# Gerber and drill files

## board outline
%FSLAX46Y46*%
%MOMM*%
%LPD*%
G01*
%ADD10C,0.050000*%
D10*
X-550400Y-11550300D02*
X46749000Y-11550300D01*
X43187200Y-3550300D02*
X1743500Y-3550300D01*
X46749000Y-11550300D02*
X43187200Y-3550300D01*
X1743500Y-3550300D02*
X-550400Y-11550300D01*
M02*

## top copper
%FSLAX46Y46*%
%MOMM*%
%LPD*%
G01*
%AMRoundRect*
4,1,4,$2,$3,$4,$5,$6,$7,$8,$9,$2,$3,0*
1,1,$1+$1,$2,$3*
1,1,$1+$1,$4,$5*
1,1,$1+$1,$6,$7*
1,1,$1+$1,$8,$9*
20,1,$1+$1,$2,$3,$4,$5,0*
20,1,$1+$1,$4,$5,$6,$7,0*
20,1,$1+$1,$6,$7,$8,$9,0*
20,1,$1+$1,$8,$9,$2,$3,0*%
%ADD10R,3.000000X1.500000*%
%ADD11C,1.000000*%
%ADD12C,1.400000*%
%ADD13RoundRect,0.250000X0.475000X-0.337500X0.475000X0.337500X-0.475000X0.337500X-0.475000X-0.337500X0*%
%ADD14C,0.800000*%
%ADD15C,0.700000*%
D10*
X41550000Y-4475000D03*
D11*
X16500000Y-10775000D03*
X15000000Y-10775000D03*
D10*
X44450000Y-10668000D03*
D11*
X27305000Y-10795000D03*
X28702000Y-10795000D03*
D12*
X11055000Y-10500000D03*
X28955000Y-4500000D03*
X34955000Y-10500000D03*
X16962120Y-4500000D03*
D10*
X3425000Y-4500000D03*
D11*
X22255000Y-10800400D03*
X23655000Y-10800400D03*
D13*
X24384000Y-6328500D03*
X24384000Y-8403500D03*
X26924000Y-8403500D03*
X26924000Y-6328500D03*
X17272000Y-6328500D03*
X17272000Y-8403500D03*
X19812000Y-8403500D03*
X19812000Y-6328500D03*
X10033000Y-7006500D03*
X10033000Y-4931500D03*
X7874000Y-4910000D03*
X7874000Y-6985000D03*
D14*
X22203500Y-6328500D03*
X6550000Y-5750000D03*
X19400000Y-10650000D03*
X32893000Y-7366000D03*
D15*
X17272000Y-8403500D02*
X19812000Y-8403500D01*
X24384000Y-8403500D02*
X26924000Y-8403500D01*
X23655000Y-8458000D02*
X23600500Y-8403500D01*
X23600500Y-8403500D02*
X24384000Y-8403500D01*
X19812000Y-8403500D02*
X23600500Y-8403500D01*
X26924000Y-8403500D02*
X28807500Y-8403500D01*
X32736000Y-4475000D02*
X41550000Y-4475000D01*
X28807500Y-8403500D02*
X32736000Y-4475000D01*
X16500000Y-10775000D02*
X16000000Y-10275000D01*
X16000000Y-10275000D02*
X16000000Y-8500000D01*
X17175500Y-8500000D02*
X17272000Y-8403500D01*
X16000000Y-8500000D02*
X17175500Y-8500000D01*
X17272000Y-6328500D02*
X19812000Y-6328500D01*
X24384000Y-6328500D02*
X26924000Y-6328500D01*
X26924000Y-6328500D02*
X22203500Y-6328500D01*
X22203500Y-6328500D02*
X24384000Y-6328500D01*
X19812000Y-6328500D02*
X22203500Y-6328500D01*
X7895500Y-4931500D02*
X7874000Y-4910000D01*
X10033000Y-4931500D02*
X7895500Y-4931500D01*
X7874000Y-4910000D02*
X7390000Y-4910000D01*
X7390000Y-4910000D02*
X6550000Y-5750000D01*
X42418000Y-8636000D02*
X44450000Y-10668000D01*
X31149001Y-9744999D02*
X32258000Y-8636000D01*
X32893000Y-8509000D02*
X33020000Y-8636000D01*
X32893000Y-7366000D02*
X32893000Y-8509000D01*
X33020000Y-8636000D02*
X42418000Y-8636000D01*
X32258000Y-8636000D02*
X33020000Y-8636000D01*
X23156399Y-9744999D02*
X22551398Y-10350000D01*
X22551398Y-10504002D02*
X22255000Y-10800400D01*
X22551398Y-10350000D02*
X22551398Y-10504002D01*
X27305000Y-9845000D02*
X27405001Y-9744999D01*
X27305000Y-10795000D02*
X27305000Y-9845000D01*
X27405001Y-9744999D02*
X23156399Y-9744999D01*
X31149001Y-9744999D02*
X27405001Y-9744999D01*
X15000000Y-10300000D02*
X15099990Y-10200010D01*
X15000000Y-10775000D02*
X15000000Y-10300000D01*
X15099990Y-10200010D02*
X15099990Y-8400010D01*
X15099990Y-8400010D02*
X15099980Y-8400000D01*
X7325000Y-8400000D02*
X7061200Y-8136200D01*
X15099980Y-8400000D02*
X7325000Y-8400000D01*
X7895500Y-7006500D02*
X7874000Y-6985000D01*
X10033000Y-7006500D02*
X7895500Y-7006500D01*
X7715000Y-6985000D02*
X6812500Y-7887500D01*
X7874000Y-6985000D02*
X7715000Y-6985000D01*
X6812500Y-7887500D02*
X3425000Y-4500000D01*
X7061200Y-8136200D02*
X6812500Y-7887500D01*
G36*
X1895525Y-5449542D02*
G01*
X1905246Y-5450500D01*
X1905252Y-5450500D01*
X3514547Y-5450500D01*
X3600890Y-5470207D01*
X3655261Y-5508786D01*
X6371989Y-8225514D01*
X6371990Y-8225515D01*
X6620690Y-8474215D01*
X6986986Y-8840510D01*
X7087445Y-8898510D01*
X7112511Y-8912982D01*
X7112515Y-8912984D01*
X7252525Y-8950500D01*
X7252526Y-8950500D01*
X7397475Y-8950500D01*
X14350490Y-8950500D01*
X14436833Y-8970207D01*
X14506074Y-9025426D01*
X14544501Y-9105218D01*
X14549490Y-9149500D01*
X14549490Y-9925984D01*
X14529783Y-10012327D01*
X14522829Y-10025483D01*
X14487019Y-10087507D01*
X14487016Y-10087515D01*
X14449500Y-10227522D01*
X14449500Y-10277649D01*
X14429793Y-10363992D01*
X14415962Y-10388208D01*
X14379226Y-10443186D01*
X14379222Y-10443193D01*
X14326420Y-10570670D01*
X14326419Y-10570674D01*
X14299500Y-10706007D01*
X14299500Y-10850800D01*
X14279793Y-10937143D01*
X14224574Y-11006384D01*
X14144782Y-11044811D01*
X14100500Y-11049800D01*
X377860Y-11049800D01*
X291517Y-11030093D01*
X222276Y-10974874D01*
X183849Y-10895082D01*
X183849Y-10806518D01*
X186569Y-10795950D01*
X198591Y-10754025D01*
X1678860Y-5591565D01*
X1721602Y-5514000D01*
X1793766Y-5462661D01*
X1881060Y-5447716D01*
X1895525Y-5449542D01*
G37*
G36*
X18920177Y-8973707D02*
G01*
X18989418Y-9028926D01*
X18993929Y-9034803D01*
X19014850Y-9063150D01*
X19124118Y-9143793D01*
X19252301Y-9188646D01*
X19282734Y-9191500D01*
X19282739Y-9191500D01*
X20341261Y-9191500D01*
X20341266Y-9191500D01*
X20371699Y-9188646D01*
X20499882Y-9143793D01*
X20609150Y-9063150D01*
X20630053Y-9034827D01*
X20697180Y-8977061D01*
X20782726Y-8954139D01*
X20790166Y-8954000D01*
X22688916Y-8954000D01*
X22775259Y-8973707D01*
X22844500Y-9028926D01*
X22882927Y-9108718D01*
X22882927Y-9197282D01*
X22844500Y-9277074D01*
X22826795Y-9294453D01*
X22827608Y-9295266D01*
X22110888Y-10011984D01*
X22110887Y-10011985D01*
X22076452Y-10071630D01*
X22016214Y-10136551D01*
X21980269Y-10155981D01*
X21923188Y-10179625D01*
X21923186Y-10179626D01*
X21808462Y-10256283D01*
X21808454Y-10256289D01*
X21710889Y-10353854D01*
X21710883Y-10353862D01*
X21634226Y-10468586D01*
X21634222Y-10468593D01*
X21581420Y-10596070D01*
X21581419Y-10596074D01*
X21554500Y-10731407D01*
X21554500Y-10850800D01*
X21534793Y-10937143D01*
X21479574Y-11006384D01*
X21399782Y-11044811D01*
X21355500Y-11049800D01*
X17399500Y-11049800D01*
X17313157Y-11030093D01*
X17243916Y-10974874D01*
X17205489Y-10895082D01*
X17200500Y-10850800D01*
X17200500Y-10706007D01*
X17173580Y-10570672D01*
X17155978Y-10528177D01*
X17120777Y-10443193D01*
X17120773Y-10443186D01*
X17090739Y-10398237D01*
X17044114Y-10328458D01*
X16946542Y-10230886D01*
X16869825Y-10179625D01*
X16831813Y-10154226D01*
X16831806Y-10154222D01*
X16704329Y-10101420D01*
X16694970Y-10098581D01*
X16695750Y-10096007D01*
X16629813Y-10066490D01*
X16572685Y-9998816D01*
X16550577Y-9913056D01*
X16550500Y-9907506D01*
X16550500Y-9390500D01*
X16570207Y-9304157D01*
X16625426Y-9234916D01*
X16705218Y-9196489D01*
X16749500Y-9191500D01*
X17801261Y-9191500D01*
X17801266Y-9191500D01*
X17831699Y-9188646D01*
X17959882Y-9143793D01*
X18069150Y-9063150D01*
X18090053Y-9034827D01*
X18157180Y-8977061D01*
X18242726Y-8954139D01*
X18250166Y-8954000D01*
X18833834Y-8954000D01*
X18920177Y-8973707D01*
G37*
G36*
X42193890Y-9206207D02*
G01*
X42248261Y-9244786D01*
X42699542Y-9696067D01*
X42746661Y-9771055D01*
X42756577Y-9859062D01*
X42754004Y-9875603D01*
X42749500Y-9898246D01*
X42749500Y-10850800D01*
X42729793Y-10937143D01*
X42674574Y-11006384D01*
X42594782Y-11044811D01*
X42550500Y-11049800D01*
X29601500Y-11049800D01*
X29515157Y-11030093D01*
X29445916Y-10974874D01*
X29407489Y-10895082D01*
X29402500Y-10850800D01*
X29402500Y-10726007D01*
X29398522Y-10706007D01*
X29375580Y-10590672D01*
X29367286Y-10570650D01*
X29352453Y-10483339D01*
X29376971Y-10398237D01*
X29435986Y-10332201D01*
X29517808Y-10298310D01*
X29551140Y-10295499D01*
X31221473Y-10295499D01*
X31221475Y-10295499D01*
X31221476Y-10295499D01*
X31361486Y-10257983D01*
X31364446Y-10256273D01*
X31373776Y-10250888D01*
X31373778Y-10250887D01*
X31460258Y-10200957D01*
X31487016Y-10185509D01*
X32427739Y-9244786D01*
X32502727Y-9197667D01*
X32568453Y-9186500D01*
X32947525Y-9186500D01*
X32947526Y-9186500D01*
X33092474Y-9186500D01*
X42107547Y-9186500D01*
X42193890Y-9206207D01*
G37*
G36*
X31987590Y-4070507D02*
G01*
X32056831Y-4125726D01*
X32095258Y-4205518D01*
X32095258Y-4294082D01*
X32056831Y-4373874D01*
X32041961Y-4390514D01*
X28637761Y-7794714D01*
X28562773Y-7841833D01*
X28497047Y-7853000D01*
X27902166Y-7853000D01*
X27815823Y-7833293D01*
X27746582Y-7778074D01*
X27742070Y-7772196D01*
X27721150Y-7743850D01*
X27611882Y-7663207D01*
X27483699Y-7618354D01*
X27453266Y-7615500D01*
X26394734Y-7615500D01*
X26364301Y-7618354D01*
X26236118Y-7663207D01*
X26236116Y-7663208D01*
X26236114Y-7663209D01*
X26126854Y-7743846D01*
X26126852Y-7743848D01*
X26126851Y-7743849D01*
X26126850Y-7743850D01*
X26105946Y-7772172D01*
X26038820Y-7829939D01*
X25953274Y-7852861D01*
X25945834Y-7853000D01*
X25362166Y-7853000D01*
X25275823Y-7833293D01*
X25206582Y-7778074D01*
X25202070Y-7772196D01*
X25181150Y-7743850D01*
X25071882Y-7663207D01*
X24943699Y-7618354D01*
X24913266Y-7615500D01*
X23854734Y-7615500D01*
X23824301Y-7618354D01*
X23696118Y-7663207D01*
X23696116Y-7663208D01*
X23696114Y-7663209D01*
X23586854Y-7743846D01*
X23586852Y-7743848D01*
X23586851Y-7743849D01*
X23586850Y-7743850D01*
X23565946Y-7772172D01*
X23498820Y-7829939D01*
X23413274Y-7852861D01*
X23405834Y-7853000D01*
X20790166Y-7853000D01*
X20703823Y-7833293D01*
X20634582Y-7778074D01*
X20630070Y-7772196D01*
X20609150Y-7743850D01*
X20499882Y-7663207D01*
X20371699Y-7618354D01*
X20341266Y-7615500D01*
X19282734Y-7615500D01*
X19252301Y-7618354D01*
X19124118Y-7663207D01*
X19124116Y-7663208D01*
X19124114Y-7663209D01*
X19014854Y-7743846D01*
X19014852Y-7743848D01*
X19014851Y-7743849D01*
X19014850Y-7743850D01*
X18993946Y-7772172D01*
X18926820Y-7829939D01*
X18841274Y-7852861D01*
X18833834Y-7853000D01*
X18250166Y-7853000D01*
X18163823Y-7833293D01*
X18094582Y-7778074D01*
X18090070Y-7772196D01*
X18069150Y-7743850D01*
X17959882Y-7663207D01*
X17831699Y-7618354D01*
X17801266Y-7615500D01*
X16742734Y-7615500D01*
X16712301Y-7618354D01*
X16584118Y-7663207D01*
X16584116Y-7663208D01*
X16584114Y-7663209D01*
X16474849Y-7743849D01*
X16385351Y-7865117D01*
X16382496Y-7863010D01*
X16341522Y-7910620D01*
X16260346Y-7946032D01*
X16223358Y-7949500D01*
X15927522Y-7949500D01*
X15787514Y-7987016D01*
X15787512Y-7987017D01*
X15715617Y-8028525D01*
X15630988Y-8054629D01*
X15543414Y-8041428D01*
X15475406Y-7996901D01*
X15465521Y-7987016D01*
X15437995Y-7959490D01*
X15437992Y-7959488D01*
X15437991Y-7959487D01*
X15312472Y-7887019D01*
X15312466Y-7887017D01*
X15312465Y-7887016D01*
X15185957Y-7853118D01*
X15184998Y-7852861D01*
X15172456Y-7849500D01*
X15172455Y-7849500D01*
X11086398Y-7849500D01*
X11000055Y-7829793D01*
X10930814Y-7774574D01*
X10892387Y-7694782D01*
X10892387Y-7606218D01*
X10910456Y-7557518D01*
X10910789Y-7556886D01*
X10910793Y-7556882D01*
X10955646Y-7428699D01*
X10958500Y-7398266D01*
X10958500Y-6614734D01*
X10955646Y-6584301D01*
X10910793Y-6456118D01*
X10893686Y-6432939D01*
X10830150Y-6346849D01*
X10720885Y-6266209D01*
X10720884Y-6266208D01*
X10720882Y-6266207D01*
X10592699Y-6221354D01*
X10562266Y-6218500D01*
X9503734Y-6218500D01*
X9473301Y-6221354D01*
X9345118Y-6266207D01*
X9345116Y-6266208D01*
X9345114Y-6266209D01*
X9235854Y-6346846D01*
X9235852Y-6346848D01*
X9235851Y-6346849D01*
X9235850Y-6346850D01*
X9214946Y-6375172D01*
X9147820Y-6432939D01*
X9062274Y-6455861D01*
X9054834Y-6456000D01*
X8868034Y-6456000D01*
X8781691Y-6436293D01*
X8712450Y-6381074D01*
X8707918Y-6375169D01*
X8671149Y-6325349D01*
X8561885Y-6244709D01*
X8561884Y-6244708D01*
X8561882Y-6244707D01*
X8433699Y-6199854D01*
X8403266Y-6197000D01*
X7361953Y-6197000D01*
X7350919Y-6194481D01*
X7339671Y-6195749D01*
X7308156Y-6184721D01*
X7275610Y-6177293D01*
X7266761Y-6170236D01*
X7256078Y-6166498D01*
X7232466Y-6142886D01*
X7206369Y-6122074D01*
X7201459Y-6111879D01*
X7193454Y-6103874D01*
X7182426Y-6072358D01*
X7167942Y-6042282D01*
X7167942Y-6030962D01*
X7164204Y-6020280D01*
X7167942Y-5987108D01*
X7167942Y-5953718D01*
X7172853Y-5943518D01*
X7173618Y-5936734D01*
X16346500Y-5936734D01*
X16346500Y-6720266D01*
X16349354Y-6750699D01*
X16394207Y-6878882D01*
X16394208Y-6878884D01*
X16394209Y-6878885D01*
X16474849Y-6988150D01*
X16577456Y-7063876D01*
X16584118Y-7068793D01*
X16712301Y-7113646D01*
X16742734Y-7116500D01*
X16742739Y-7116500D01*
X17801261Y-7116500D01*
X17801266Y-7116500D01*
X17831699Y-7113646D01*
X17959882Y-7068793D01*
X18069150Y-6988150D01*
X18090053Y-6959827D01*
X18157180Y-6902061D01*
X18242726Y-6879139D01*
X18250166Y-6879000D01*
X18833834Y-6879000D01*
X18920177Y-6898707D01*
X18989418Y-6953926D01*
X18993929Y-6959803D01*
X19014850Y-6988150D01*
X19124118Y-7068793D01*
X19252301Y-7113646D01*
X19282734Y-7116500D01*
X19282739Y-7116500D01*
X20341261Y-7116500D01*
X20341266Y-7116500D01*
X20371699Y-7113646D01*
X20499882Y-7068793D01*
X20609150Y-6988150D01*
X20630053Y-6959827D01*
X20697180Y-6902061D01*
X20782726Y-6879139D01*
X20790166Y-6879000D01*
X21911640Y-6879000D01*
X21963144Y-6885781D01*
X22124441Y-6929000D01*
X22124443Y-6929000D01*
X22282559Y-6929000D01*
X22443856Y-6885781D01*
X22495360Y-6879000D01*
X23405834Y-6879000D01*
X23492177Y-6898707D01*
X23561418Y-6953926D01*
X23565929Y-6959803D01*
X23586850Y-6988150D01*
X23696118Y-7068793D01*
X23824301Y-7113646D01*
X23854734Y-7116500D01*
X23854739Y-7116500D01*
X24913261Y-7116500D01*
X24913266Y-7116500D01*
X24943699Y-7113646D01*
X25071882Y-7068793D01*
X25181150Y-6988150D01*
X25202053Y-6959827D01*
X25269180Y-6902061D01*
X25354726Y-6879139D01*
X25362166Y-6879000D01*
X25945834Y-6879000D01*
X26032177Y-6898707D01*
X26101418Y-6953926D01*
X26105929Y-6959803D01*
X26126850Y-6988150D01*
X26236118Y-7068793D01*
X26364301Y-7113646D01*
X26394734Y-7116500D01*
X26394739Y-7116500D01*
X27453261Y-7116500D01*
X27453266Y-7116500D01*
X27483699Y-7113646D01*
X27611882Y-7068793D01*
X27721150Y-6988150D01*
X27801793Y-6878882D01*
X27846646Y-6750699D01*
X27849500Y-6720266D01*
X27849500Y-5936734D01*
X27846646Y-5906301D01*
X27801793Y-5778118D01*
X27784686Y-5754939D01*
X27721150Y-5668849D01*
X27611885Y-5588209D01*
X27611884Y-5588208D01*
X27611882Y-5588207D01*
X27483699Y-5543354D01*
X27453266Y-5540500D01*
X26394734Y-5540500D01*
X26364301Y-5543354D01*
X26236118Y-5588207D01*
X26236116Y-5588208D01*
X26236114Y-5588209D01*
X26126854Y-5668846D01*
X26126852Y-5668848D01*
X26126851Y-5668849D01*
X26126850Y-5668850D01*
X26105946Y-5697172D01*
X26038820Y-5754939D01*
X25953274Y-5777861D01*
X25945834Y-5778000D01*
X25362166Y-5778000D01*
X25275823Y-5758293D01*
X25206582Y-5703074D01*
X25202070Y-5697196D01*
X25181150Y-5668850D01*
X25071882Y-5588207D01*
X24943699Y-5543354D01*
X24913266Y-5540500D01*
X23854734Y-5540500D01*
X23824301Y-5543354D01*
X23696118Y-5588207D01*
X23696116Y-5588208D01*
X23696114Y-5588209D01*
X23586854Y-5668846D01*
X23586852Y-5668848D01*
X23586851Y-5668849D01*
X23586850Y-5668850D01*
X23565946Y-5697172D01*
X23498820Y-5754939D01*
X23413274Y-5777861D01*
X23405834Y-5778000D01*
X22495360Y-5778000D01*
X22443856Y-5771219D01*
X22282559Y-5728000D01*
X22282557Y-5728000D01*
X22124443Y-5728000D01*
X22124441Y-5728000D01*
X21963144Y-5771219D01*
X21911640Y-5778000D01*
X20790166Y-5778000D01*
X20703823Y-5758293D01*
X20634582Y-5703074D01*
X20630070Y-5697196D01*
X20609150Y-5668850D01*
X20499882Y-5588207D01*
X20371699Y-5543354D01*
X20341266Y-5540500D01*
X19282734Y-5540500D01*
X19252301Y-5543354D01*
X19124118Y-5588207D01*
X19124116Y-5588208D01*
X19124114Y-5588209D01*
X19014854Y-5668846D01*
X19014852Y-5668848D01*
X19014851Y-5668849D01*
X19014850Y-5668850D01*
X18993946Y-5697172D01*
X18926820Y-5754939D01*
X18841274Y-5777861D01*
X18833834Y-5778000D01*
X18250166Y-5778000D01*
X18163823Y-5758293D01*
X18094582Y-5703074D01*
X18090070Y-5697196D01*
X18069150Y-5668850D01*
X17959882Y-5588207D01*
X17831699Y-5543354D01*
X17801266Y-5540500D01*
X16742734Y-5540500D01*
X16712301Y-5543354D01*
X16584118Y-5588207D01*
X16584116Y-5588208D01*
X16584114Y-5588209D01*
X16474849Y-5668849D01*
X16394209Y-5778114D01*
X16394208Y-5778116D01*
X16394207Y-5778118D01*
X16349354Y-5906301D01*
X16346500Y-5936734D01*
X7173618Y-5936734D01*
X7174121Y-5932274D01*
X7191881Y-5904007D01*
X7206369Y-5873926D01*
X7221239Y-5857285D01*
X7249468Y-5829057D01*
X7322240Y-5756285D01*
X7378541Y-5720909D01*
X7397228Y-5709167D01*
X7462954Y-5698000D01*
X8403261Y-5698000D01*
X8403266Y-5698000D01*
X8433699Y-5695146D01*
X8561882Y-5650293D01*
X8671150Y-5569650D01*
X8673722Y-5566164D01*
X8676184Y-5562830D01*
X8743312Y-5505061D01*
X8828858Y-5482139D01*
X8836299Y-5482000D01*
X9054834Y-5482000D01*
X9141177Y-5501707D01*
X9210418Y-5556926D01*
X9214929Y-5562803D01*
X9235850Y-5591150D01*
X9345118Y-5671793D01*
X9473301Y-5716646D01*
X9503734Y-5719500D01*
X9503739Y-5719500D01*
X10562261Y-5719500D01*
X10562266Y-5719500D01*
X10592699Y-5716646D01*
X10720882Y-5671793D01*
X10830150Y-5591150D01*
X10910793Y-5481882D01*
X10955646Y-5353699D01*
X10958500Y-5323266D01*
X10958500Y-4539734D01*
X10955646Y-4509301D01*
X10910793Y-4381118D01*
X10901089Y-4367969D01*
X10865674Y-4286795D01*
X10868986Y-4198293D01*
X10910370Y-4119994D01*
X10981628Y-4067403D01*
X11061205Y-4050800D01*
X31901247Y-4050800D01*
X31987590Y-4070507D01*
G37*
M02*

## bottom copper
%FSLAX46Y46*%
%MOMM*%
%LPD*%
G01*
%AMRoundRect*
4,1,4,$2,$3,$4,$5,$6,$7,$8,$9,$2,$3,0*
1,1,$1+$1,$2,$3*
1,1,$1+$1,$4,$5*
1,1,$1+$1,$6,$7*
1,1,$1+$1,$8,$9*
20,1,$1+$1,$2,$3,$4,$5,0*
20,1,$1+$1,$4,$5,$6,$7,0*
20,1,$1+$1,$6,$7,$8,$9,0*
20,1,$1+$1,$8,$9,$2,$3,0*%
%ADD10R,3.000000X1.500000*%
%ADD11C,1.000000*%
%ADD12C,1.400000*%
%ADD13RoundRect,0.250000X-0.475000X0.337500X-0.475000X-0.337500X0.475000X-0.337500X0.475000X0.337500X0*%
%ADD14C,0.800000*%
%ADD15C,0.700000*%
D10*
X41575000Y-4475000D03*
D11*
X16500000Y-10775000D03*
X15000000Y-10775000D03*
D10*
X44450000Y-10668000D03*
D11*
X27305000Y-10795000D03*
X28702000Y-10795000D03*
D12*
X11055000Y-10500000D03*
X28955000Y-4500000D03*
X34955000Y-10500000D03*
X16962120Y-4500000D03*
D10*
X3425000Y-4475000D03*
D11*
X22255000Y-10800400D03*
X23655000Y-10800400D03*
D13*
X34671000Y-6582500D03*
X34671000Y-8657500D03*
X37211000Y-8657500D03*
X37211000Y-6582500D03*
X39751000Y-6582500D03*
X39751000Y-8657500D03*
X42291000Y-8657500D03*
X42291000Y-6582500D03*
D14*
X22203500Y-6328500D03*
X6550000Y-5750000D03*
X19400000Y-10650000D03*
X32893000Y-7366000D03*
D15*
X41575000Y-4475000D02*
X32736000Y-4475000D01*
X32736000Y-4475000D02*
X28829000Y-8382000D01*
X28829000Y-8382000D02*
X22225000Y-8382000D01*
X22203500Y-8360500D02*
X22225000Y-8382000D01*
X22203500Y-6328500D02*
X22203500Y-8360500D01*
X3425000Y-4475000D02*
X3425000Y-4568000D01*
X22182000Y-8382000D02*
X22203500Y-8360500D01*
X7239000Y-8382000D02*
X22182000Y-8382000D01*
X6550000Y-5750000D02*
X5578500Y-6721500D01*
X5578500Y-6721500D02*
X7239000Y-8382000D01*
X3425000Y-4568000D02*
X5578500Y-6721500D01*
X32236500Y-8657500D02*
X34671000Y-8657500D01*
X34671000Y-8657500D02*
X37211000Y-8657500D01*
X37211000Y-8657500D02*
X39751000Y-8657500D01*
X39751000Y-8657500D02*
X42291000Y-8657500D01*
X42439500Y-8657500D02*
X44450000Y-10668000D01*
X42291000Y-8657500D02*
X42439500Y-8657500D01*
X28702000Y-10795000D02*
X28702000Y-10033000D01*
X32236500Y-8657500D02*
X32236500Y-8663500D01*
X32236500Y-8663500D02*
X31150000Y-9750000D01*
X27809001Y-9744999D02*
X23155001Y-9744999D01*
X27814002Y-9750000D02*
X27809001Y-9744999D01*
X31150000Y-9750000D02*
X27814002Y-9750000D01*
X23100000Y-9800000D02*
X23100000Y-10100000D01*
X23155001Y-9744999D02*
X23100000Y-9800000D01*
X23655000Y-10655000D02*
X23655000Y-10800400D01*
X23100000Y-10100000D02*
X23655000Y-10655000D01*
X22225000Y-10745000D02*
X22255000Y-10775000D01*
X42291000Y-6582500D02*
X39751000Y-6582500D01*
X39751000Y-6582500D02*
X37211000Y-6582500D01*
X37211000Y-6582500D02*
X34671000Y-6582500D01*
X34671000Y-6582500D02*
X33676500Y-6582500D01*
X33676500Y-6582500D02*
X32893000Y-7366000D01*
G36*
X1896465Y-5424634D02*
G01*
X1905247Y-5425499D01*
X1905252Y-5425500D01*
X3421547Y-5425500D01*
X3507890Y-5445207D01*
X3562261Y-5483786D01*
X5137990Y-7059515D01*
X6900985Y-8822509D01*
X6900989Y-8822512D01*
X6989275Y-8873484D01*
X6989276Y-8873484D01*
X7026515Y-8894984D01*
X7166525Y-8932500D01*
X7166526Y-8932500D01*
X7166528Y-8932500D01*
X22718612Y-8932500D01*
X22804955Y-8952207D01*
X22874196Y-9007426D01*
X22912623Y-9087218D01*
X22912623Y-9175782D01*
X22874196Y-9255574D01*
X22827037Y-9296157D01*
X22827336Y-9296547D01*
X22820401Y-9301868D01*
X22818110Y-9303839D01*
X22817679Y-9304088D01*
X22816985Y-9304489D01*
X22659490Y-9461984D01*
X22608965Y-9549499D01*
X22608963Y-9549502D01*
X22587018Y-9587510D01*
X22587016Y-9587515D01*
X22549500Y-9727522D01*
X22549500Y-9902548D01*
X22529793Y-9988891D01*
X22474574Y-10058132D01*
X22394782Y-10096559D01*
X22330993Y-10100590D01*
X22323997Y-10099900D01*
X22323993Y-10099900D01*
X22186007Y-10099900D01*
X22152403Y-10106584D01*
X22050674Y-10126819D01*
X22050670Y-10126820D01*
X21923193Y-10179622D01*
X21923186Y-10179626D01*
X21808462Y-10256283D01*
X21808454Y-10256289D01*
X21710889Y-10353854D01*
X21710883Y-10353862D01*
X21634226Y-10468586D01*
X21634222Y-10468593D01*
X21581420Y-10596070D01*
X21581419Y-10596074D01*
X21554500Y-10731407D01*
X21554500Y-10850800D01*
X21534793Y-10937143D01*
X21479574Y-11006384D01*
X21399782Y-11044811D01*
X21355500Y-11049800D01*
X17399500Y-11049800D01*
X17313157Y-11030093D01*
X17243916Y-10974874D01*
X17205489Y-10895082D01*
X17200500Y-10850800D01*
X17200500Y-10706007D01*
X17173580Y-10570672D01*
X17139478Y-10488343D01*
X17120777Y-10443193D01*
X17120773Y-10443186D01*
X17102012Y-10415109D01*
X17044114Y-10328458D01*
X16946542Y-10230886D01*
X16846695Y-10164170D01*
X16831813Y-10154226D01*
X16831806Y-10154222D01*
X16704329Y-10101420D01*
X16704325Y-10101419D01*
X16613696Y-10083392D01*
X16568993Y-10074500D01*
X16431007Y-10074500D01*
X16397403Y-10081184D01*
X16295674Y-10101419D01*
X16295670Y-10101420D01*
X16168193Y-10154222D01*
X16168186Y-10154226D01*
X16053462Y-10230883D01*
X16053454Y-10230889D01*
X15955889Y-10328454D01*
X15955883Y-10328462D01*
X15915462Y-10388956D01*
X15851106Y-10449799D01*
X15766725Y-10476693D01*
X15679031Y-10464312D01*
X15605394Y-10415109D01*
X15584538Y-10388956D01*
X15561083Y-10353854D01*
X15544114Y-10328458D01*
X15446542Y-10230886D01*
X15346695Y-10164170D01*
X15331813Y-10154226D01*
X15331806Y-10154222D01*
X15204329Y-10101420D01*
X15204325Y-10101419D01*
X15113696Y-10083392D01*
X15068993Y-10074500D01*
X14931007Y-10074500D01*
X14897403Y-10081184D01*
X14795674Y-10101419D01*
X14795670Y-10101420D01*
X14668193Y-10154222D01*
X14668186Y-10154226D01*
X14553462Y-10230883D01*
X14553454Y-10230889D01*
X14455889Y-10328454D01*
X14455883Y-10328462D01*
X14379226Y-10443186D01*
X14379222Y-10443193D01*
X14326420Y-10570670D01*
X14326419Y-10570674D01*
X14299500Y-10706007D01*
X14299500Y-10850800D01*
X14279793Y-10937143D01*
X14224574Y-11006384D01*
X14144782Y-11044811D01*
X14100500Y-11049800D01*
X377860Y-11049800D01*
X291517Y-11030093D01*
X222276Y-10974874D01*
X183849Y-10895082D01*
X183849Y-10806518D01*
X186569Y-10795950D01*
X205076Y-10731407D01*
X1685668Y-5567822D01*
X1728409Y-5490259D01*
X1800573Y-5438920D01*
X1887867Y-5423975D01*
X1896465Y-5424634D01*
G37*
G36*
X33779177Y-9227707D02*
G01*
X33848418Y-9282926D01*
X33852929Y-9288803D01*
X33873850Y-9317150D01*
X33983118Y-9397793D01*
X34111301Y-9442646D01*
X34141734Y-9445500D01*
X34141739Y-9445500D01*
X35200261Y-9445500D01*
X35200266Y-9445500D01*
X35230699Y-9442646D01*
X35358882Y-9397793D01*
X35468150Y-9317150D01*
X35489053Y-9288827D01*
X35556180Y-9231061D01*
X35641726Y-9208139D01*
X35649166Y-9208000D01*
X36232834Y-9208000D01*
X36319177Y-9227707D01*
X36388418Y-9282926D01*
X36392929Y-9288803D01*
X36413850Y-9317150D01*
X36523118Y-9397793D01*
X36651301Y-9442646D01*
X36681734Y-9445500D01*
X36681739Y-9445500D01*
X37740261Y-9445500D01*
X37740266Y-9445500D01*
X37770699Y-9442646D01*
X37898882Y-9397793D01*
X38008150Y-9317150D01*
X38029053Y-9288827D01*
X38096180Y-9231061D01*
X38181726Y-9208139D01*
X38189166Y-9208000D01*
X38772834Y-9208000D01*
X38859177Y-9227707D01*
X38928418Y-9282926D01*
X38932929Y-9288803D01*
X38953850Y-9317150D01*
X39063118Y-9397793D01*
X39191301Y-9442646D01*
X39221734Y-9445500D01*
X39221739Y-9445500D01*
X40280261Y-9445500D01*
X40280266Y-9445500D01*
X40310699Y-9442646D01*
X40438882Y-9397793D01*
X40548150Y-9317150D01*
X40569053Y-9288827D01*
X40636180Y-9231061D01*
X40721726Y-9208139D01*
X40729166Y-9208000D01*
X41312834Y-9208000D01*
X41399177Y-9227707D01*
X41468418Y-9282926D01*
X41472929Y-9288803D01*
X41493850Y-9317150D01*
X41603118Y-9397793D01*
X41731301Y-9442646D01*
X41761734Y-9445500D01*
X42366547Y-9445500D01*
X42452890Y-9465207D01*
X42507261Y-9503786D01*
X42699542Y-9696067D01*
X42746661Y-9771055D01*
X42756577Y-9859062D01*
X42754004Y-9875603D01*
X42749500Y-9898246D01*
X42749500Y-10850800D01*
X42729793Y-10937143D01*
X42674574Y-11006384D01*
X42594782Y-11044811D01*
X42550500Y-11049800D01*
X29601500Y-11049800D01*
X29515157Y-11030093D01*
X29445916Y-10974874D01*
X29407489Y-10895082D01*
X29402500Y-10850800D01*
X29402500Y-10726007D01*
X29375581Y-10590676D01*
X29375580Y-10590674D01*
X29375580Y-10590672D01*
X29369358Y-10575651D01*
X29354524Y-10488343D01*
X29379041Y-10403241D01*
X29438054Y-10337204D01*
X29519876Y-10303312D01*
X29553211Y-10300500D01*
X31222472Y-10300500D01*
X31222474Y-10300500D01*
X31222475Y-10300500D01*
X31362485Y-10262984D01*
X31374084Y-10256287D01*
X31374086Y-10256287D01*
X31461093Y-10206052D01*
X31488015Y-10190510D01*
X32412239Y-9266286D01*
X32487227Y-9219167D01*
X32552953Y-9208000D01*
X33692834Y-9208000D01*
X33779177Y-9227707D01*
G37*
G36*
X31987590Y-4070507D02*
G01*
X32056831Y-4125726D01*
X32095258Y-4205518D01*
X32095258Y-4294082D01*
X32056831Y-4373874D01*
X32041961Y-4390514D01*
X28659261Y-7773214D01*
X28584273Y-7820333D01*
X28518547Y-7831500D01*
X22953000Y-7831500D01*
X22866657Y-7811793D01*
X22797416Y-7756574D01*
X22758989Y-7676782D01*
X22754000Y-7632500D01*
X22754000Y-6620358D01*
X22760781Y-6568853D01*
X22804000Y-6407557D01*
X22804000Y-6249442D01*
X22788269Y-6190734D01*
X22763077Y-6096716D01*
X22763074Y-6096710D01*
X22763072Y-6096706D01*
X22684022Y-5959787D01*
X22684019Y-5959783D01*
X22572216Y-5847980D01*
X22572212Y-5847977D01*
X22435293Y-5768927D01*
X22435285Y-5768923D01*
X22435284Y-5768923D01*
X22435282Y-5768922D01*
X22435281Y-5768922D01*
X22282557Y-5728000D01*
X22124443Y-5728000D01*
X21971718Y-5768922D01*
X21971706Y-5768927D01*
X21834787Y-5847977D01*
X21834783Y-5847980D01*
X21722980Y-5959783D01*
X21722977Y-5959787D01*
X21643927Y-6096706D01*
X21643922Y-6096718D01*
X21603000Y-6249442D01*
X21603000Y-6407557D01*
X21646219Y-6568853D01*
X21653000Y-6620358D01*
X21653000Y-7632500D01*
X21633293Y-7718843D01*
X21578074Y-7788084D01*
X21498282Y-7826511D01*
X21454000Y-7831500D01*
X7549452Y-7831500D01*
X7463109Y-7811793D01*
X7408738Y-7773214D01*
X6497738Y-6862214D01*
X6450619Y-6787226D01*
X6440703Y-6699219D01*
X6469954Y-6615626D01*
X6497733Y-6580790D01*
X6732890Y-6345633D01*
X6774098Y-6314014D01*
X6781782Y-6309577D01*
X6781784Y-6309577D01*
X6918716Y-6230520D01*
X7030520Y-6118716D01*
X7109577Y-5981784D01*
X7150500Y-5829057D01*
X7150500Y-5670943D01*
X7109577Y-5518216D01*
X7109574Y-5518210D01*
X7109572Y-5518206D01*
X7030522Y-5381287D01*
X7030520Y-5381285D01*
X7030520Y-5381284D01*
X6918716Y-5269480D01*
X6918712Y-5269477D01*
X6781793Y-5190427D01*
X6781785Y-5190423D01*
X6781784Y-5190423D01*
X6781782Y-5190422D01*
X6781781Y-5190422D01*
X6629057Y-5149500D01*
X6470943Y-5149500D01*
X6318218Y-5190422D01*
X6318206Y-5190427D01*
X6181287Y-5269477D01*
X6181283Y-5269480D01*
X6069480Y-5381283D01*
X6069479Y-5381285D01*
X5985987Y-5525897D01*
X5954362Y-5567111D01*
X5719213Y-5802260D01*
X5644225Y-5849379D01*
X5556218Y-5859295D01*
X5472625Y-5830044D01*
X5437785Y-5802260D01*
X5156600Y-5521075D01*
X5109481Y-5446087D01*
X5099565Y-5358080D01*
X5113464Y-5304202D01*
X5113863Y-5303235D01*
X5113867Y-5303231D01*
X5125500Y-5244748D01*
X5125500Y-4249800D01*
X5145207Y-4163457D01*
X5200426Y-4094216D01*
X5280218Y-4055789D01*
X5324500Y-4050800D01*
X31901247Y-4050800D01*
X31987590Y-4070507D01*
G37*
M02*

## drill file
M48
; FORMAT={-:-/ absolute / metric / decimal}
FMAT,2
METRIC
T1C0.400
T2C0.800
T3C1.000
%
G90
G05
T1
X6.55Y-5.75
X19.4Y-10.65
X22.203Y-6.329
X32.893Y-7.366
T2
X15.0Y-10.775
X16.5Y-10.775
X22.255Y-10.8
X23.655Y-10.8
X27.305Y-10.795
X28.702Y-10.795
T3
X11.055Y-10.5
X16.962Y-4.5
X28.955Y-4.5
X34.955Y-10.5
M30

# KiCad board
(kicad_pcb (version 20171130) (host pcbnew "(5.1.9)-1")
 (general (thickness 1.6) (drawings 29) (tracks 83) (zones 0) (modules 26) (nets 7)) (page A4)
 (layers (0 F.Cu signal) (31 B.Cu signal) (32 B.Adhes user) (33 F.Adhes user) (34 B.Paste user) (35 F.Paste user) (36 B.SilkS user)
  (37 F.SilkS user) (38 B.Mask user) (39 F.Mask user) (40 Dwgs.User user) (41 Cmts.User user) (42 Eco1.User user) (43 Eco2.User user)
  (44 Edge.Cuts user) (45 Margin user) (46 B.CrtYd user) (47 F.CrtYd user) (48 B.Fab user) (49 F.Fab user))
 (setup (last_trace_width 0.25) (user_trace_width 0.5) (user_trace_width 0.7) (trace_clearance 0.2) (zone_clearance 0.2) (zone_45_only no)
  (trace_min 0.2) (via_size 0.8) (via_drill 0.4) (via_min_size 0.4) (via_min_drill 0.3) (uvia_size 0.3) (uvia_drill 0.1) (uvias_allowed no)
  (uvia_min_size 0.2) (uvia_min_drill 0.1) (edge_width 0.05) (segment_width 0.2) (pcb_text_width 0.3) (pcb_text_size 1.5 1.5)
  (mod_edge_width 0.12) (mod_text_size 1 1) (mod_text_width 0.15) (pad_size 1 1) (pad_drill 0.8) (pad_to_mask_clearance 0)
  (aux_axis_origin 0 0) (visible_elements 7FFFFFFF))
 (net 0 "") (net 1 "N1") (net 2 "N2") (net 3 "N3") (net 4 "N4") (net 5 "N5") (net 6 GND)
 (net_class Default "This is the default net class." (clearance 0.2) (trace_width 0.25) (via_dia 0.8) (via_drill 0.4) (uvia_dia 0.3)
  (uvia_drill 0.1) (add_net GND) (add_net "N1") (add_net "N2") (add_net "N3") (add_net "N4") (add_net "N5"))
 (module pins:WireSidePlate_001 (layer F.Cu) (at 41.55 2.275)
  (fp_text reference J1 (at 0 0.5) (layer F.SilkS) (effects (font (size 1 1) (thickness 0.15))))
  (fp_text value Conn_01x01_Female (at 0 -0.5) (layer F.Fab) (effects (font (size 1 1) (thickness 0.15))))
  (pad 1 smd rect (at 0 2.2) (size 3 1.5) (layers F.Cu F.Paste F.Mask) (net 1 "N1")))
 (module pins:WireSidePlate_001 (layer B.Cu) (at 41.575 6.675)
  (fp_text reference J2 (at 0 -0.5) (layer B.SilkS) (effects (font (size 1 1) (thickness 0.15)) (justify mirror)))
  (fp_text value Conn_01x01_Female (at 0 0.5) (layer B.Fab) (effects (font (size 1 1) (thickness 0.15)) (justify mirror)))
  (pad 1 smd rect (at 0 -2.2) (size 3 1.5) (layers B.Cu B.Paste B.Mask) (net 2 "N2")))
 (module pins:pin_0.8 (layer F.Cu) (at 23.655 10.775 270)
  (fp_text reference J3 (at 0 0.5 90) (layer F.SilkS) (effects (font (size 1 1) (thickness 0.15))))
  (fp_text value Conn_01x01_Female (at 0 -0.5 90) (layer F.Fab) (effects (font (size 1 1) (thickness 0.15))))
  (pad 1 thru_hole circle (at 0 7.155 270) (size 1 1) (drill 0.8) (layers *.Cu *.Mask) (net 1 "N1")))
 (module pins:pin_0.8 (layer F.Cu) (at 21.65 10.775 270)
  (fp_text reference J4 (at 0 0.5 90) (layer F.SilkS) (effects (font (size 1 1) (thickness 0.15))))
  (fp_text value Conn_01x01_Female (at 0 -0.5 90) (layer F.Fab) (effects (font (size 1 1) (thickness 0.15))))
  (pad 1 thru_hole circle (at 0 6.65 270) (size 1 1) (drill 0.8) (layers *.Cu *.Mask) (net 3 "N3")))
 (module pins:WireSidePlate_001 (layer F.Cu) (at 44.45 8.468)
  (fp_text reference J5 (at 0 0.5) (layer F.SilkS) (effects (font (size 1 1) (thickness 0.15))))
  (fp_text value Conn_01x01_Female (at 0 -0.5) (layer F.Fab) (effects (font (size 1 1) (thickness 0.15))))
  (pad 1 smd rect (at 0 2.2) (size 3 1.5) (layers F.Cu F.Paste F.Mask) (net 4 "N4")))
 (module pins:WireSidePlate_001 (layer B.Cu) (at 44.45 12.868)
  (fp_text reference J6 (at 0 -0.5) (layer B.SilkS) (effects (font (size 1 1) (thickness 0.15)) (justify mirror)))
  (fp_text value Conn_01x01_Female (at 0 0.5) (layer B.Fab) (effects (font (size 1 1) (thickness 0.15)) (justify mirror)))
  (pad 1 smd rect (at 0 -2.2) (size 3 1.5) (layers B.Cu B.Paste B.Mask) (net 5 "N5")))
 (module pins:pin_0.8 (layer F.Cu) (at 27.305 9.195)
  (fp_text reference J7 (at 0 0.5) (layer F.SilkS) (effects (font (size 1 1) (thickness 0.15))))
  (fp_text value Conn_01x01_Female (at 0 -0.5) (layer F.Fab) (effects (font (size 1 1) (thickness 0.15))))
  (pad 1 thru_hole circle (at 0 1.6) (size 1 1) (drill 0.8) (layers *.Cu *.Mask) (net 4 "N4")))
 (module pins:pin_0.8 (layer F.Cu) (at 28.702 9.195)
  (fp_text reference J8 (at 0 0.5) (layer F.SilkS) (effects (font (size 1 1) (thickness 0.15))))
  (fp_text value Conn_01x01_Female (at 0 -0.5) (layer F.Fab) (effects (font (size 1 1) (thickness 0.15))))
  (pad 1 thru_hole circle (at 0 1.6) (size 1 1) (drill 0.8) (layers *.Cu *.Mask) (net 5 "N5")))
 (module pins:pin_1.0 (layer F.Cu) (at 31.195 22.195)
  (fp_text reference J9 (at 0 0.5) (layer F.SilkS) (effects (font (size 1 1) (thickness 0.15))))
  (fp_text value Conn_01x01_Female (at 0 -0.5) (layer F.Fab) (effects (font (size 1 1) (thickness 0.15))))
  (pad 1 thru_hole circle (at -20.14 -11.695) (size 1.4 1.4) (drill 1) (layers *.Cu *.Mask) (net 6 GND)))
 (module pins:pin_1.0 (layer F.Cu) (at 28.855 2.5)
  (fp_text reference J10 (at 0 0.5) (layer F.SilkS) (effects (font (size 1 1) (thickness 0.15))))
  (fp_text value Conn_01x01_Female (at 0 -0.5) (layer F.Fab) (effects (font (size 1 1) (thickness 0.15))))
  (pad 1 thru_hole circle (at 0.1 2) (size 1.4 1.4) (drill 1) (layers *.Cu *.Mask) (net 6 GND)))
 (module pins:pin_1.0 (layer F.Cu) (at 30.385 26.395)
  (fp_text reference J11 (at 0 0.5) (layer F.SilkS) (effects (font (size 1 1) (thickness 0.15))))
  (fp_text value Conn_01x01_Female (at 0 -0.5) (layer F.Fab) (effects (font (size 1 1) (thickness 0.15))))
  (pad 1 thru_hole circle (at 4.57 -15.895) (size 1.4 1.4) (drill 1) (layers *.Cu *.Mask) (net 6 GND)))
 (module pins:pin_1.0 (layer F.Cu) (at 16.86212 2.5)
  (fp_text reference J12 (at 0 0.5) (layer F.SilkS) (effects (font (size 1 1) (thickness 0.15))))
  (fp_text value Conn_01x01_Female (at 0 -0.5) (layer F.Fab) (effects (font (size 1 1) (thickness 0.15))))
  (pad 1 thru_hole circle (at 0.1 2) (size 1.4 1.4) (drill 1) (layers *.Cu *.Mask) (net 6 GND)))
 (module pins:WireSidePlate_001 (layer F.Cu) (at 3.425 2.3)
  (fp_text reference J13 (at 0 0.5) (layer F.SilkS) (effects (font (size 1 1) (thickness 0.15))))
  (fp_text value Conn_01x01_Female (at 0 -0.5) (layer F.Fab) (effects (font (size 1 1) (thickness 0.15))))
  (pad 1 smd rect (at 0 2.2) (size 3 1.5) (layers F.Cu F.Paste F.Mask) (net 3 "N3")))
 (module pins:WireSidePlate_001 (layer B.Cu) (at 3.425 6.675)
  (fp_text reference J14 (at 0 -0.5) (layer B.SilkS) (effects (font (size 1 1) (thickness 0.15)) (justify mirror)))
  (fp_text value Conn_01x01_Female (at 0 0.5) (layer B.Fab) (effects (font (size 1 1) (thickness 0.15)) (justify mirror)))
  (pad 1 smd rect (at 0 -2.2) (size 3 1.5) (layers B.Cu B.Paste B.Mask) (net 2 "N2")))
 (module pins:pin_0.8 (layer F.Cu) (at 8.45764 9.20068)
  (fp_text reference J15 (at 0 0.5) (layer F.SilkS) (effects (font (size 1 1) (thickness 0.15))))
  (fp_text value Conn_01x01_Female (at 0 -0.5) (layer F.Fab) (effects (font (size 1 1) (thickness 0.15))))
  (pad 1 thru_hole circle (at 13.79736 1.59972) (size 1 1) (drill 0.8) (layers *.Cu *.Mask) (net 4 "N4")))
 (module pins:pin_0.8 (layer F.Cu) (at 7.0612 9.20008)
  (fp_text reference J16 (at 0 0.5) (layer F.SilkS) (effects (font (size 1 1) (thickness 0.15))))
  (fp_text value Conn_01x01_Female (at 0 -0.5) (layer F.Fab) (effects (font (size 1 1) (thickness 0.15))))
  (pad 1 thru_hole circle (at 16.5938 1.60032) (size 1 1) (drill 0.8) (layers *.Cu *.Mask) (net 5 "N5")))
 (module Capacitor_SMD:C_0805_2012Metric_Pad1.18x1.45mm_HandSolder (layer B.Cu) (at 34.671 7.62 270)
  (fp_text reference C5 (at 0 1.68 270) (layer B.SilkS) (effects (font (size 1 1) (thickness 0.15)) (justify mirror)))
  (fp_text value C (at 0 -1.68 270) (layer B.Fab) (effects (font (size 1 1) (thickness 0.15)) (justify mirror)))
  (pad 1 smd roundrect (at -1.0375 0 270) (size 1.175 1.45) (layers B.Cu B.Paste B.Mask) (roundrect_rratio 0.2127659574468085) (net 4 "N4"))
  (pad 2 smd roundrect (at 1.0375 0 270) (size 1.175 1.45) (layers B.Cu B.Paste B.Mask) (roundrect_rratio 0.2127659574468085) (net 5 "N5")))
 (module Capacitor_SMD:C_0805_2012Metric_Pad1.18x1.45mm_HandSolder (layer B.Cu) (at 37.211 7.62 270)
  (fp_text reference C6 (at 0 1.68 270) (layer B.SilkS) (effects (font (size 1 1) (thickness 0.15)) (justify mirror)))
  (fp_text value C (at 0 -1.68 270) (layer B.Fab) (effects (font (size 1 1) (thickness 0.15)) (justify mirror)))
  (pad 2 smd roundrect (at 1.0375 0 270) (size 1.175 1.45) (layers B.Cu B.Paste B.Mask) (roundrect_rratio 0.2127659574468085) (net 5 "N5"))
  (pad 1 smd roundrect (at -1.0375 0 270) (size 1.175 1.45) (layers B.Cu B.Paste B.Mask) (roundrect_rratio 0.2127659574468085) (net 4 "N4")))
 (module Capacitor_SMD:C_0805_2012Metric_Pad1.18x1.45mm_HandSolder (layer B.Cu) (at 39.751 7.62 270)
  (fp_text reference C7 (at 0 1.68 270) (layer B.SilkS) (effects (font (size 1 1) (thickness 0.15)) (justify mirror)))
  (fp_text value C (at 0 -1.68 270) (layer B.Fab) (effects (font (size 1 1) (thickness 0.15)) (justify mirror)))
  (pad 1 smd roundrect (at -1.0375 0 270) (size 1.175 1.45) (layers B.Cu B.Paste B.Mask) (roundrect_rratio 0.2127659574468085) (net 4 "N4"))
  (pad 2 smd roundrect (at 1.0375 0 270) (size 1.175 1.45) (layers B.Cu B.Paste B.Mask) (roundrect_rratio 0.2127659574468085) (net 5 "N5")))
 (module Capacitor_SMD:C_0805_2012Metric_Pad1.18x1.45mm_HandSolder (layer B.Cu) (at 42.291 7.62 270)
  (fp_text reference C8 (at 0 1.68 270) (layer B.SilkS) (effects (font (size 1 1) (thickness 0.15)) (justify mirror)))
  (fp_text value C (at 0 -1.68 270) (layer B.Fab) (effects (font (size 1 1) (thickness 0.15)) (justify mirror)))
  (pad 2 smd roundrect (at 1.0375 0 270) (size 1.175 1.45) (layers B.Cu B.Paste B.Mask) (roundrect_rratio 0.2127659574468085) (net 5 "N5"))
  (pad 1 smd roundrect (at -1.0375 0 270) (size 1.175 1.45) (layers B.Cu B.Paste B.Mask) (roundrect_rratio 0.2127659574468085) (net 4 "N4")))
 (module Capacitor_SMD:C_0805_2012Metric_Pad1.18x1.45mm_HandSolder (layer F.Cu) (at 24.384 7.366 90)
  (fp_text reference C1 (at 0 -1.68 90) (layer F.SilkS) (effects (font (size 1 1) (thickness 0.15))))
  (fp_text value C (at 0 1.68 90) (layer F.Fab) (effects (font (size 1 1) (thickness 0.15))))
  (pad 2 smd roundrect (at 1.0375 0 90) (size 1.175 1.45) (layers F.Cu F.Paste F.Mask) (roundrect_rratio 0.2127659574468085) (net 2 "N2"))
  (pad 1 smd roundrect (at -1.0375 0 90) (size 1.175 1.45) (layers F.Cu F.Paste F.Mask) (roundrect_rratio 0.2127659574468085) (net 1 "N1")))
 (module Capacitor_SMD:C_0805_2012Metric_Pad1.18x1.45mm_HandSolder (layer F.Cu) (at 26.924 7.366 90)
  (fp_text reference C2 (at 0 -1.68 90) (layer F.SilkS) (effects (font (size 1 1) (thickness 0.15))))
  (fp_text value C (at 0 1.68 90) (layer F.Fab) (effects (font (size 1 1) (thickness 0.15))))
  (pad 1 smd roundrect (at -1.0375 0 90) (size 1.175 1.45) (layers F.Cu F.Paste F.Mask) (roundrect_rratio 0.2127659574468085) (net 1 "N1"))
  (pad 2 smd roundrect (at 1.0375 0 90) (size 1.175 1.45) (layers F.Cu F.Paste F.Mask) (roundrect_rratio 0.2127659574468085) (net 2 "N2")))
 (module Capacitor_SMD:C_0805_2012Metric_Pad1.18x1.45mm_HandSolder (layer F.Cu) (at 17.272 7.366 90)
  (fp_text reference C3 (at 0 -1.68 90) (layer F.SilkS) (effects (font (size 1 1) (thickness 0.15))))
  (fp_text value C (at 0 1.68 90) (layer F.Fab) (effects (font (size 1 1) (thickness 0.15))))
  (pad 2 smd roundrect (at 1.0375 0 90) (size 1.175 1.45) (layers F.Cu F.Paste F.Mask) (roundrect_rratio 0.2127659574468085) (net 2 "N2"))
  (pad 1 smd roundrect (at -1.0375 0 90) (size 1.175 1.45) (layers F.Cu F.Paste F.Mask) (roundrect_rratio 0.2127659574468085) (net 1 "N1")))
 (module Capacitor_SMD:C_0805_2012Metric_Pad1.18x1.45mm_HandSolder (layer F.Cu) (at 19.812 7.366 90)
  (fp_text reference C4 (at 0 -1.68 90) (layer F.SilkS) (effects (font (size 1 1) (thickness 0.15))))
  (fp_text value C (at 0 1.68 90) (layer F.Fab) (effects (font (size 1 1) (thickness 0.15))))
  (pad 1 smd roundrect (at -1.0375 0 90) (size 1.175 1.45) (layers F.Cu F.Paste F.Mask) (roundrect_rratio 0.2127659574468085) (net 1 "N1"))
  (pad 2 smd roundrect (at 1.0375 0 90) (size 1.175 1.45) (layers F.Cu F.Paste F.Mask) (roundrect_rratio 0.2127659574468085) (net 2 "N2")))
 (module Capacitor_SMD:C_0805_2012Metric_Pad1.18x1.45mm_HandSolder (layer F.Cu) (at 10.033 5.969 90)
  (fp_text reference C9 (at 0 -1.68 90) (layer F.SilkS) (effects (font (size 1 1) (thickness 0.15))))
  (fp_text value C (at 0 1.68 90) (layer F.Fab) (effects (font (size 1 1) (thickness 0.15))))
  (pad 1 smd roundrect (at -1.0375 0 90) (size 1.175 1.45) (layers F.Cu F.Paste F.Mask) (roundrect_rratio 0.2127659574468085) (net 3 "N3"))
  (pad 2 smd roundrect (at 1.0375 0 90) (size 1.175 1.45) (layers F.Cu F.Paste F.Mask) (roundrect_rratio 0.2127659574468085) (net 2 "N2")))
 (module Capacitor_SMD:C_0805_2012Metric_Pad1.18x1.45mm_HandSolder (layer F.Cu) (at 7.874 5.9475 90)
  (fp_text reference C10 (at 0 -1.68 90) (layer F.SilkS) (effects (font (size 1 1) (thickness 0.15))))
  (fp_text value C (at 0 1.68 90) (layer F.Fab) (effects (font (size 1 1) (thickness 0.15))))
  (pad 2 smd roundrect (at 1.0375 0 90) (size 1.175 1.45) (layers F.Cu F.Paste F.Mask) (roundrect_rratio 0.2127659574468085) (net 2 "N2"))
  (pad 1 smd roundrect (at -1.0375 0 90) (size 1.175 1.45) (layers F.Cu F.Paste F.Mask) (roundrect_rratio 0.2127659574468085) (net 3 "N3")))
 (gr_line (start -0.5504 11.5503) (end 46.749 11.5503) (layer Edge.Cuts) (width 0.05))
 (gr_line (start 43.1872 3.5503) (end 1.7435 3.5503) (layer Edge.Cuts) (width 0.05))
 (gr_line (start 46.749 11.5503) (end 43.1872 3.5503) (layer Edge.Cuts) (width 0.05))
 (gr_line (start 1.7435 3.5503) (end -0.5504 11.5503) (layer Edge.Cuts) (width 0.05))
 (segment (start 17.272 8.4035) (end 19.812 8.4035) (width 0.7) (layer F.Cu) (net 1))
 (segment (start 24.384 8.4035) (end 26.924 8.4035) (width 0.7) (layer F.Cu) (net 1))
 (segment (start 23.655 8.458) (end 23.6005 8.4035) (width 0.7) (layer F.Cu) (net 1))
 (segment (start 23.6005 8.4035) (end 24.384 8.4035) (width 0.7) (layer F.Cu) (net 1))
 (segment (start 19.812 8.4035) (end 23.6005 8.4035) (width 0.7) (layer F.Cu) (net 1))
 (segment (start 26.924 8.4035) (end 28.8075 8.4035) (width 0.7) (layer F.Cu) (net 1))
 (segment (start 32.736 4.475) (end 41.55 4.475) (width 0.7) (layer F.Cu) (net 1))
 (segment (start 28.8075 8.4035) (end 32.736 4.475) (width 0.7) (layer F.Cu) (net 1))
 (segment (start 16.5 10.775) (end 16 10.275) (width 0.7) (layer F.Cu) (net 1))
 (segment (start 16 10.275) (end 16 8.5) (width 0.7) (layer F.Cu) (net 1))
 (segment (start 17.1755 8.5) (end 17.272 8.4035) (width 0.7) (layer F.Cu) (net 1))
 (segment (start 16 8.5) (end 17.1755 8.5) (width 0.7) (layer F.Cu) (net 1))
 (segment (start 17.272 6.3285) (end 19.812 6.3285) (width 0.7) (layer F.Cu) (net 2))
 (segment (start 24.384 6.3285) (end 26.924 6.3285) (width 0.7) (layer F.Cu) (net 2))
 (segment (start 41.575 4.475) (end 32.736 4.475) (width 0.7) (layer B.Cu) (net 2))
 (segment (start 32.736 4.475) (end 28.829 8.382) (width 0.7) (layer B.Cu) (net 2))
 (segment (start 28.829 8.382) (end 22.225 8.382) (width 0.7) (layer B.Cu) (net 2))
 (segment (start 26.924 6.3285) (end 22.2035 6.3285) (width 0.7) (layer F.Cu) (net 2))
 (segment (start 22.2035 6.3285) (end 24.384 6.3285) (width 0.7) (layer F.Cu) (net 2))
 (segment (start 19.812 6.3285) (end 22.2035 6.3285) (width 0.7) (layer F.Cu) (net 2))
 (via (at 22.2035 6.3285) (size 0.8) (drill 0.4) (layers F.Cu B.Cu) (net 2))
 (segment (start 22.2035 8.3605) (end 22.225 8.382) (width 0.7) (layer B.Cu) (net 2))
 (segment (start 22.2035 6.3285) (end 22.2035 8.3605) (width 0.7) (layer B.Cu) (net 2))
 (segment (start 3.425 4.475) (end 3.425 4.568) (width 0.7) (layer B.Cu) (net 2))
 (segment (start 22.182 8.382) (end 22.2035 8.3605) (width 0.7) (layer B.Cu) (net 2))
 (segment (start 7.239 8.382) (end 22.182 8.382) (width 0.7) (layer B.Cu) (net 2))
 (segment (start 7.8955 4.9315) (end 7.874 4.91) (width 0.7) (layer F.Cu) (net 2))
 (segment (start 10.033 4.9315) (end 7.8955 4.9315) (width 0.7) (layer F.Cu) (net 2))
 (segment (start 7.874 4.91) (end 7.39 4.91) (width 0.7) (layer F.Cu) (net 2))
 (segment (start 7.39 4.91) (end 6.55 5.75) (width 0.7) (layer F.Cu) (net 2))
 (via (at 6.55 5.75) (size 0.8) (drill 0.4) (layers F.Cu B.Cu) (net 2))
 (segment (start 6.55 5.75) (end 5.5785 6.7215) (width 0.7) (layer B.Cu) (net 2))
 (segment (start 5.5785 6.7215) (end 7.239 8.382) (width 0.7) (layer B.Cu) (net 2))
 (segment (start 3.425 4.568) (end 5.5785 6.7215) (width 0.7) (layer B.Cu) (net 2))
 (via (at 19.4 10.65) (size 0.8) (drill 0.4) (layers F.Cu B.Cu) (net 6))
 (segment (start 32.2365 8.6575) (end 34.671 8.6575) (width 0.7) (layer B.Cu) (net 5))
 (segment (start 34.671 8.6575) (end 37.211 8.6575) (width 0.7) (layer B.Cu) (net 5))
 (segment (start 37.211 8.6575) (end 39.751 8.6575) (width 0.7) (layer B.Cu) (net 5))
 (segment (start 39.751 8.6575) (end 42.291 8.6575) (width 0.7) (layer B.Cu) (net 5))
 (segment (start 42.4395 8.6575) (end 44.45 10.668) (width 0.7) (layer B.Cu) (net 5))
 (segment (start 42.291 8.6575) (end 42.4395 8.6575) (width 0.7) (layer B.Cu) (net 5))
 (segment (start 28.702 10.795) (end 28.702 10.033) (width 0.7) (layer B.Cu) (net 5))
 (segment (start 32.2365 8.6575) (end 32.2365 8.6635) (width 0.7) (layer B.Cu) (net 5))
 (segment (start 32.2365 8.6635) (end 31.15 9.75) (width 0.7) (layer B.Cu) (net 5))
 (segment (start 27.809001 9.744999) (end 23.155001 9.744999) (width 0.7) (layer B.Cu) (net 5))
 (segment (start 27.814002 9.75) (end 27.809001 9.744999) (width 0.7) (layer B.Cu) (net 5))
 (segment (start 31.15 9.75) (end 27.814002 9.75) (width 0.7) (layer B.Cu) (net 5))
 (segment (start 23.1 9.8) (end 23.1 10.1) (width 0.7) (layer B.Cu) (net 5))
 (segment (start 23.155001 9.744999) (end 23.1 9.8) (width 0.7) (layer B.Cu) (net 5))
 (segment (start 23.655 10.655) (end 23.655 10.8004) (width 0.7) (layer B.Cu) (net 5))
 (segment (start 23.1 10.1) (end 23.655 10.655) (width 0.7) (layer B.Cu) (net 5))
 (segment (start 22.225 10.745) (end 22.255 10.775) (width 0.7) (layer B.Cu) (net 4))
 (segment (start 42.291 6.5825) (end 39.751 6.5825) (width 0.7) (layer B.Cu) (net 4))
 (segment (start 39.751 6.5825) (end 37.211 6.5825) (width 0.7) (layer B.Cu) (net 4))
 (segment (start 37.211 6.5825) (end 34.671 6.5825) (width 0.7) (layer B.Cu) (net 4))
 (segment (start 34.671 6.5825) (end 33.6765 6.5825) (width 0.7) (layer B.Cu) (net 4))
 (segment (start 33.6765 6.5825) (end 32.893 7.366) (width 0.7) (layer B.Cu) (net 4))
 (via (at 32.893 7.366) (size 0.8) (drill 0.4) (layers F.Cu B.Cu) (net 4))
 (segment (start 42.418 8.636) (end 44.45 10.668) (width 0.7) (layer F.Cu) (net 4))
 (segment (start 31.149001 9.744999) (end 32.258 8.636) (width 0.7) (layer F.Cu) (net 4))
 (segment (start 32.893 8.509) (end 33.02 8.636) (width 0.7) (layer F.Cu) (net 4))
 (segment (start 32.893 7.366) (end 32.893 8.509) (width 0.7) (layer F.Cu) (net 4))
 (segment (start 33.02 8.636) (end 42.418 8.636) (width 0.7) (layer F.Cu) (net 4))
 (segment (start 32.258 8.636) (end 33.02 8.636) (width 0.7) (layer F.Cu) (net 4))
 (segment (start 23.156399 9.744999) (end 22.551398 10.35) (width 0.7) (layer F.Cu) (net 4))
 (segment (start 22.551398 10.504002) (end 22.255 10.8004) (width 0.7) (layer F.Cu) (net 4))
 (segment (start 22.551398 10.35) (end 22.551398 10.504002) (width 0.7) (layer F.Cu) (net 4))
 (segment (start 27.305 9.845) (end 27.405001 9.744999) (width 0.7) (layer F.Cu) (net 4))
 (segment (start 27.305 10.795) (end 27.305 9.845) (width 0.7) (layer F.Cu) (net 4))
 (segment (start 27.405001 9.744999) (end 23.156399 9.744999) (width 0.7) (layer F.Cu) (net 4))
 (segment (start 31.149001 9.744999) (end 27.405001 9.744999) (width 0.7) (layer F.Cu) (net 4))
 (segment (start 15 10.3) (end 15.09999 10.20001) (width 0.7) (layer F.Cu) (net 3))
 (segment (start 15 10.775) (end 15 10.3) (width 0.7) (layer F.Cu) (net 3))
 (segment (start 15.09999 10.20001) (end 15.09999 8.40001) (width 0.7) (layer F.Cu) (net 3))
 (segment (start 15.09999 8.40001) (end 15.09998 8.4) (width 0.7) (layer F.Cu) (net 3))
 (segment (start 7.325 8.4) (end 7.0612 8.1362) (width 0.7) (layer F.Cu) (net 3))
 (segment (start 15.09998 8.4) (end 7.325 8.4) (width 0.7) (layer F.Cu) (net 3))
 (segment (start 7.8955 7.0065) (end 7.874 6.985) (width 0.7) (layer F.Cu) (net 3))
 (segment (start 10.033 7.0065) (end 7.8955 7.0065) (width 0.7) (layer F.Cu) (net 3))
 (segment (start 7.715 6.985) (end 6.8125 7.8875) (width 0.7) (layer F.Cu) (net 3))
 (segment (start 7.874 6.985) (end 7.715 6.985) (width 0.7) (layer F.Cu) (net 3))
 (segment (start 6.8125 7.8875) (end 3.425 4.5) (width 0.7) (layer F.Cu) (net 3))
 (segment (start 7.0612 8.1362) (end 6.8125 7.8875) (width 0.7) (layer F.Cu) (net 3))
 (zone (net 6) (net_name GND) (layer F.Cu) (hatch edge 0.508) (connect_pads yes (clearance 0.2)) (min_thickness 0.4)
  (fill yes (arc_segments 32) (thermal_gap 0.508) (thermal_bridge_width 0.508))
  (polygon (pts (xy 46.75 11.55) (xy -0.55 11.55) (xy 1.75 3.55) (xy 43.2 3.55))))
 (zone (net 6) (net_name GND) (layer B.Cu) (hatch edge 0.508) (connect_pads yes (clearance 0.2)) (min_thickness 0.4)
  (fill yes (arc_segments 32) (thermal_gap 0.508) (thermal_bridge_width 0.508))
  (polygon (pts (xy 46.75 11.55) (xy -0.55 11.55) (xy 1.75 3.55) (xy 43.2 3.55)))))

